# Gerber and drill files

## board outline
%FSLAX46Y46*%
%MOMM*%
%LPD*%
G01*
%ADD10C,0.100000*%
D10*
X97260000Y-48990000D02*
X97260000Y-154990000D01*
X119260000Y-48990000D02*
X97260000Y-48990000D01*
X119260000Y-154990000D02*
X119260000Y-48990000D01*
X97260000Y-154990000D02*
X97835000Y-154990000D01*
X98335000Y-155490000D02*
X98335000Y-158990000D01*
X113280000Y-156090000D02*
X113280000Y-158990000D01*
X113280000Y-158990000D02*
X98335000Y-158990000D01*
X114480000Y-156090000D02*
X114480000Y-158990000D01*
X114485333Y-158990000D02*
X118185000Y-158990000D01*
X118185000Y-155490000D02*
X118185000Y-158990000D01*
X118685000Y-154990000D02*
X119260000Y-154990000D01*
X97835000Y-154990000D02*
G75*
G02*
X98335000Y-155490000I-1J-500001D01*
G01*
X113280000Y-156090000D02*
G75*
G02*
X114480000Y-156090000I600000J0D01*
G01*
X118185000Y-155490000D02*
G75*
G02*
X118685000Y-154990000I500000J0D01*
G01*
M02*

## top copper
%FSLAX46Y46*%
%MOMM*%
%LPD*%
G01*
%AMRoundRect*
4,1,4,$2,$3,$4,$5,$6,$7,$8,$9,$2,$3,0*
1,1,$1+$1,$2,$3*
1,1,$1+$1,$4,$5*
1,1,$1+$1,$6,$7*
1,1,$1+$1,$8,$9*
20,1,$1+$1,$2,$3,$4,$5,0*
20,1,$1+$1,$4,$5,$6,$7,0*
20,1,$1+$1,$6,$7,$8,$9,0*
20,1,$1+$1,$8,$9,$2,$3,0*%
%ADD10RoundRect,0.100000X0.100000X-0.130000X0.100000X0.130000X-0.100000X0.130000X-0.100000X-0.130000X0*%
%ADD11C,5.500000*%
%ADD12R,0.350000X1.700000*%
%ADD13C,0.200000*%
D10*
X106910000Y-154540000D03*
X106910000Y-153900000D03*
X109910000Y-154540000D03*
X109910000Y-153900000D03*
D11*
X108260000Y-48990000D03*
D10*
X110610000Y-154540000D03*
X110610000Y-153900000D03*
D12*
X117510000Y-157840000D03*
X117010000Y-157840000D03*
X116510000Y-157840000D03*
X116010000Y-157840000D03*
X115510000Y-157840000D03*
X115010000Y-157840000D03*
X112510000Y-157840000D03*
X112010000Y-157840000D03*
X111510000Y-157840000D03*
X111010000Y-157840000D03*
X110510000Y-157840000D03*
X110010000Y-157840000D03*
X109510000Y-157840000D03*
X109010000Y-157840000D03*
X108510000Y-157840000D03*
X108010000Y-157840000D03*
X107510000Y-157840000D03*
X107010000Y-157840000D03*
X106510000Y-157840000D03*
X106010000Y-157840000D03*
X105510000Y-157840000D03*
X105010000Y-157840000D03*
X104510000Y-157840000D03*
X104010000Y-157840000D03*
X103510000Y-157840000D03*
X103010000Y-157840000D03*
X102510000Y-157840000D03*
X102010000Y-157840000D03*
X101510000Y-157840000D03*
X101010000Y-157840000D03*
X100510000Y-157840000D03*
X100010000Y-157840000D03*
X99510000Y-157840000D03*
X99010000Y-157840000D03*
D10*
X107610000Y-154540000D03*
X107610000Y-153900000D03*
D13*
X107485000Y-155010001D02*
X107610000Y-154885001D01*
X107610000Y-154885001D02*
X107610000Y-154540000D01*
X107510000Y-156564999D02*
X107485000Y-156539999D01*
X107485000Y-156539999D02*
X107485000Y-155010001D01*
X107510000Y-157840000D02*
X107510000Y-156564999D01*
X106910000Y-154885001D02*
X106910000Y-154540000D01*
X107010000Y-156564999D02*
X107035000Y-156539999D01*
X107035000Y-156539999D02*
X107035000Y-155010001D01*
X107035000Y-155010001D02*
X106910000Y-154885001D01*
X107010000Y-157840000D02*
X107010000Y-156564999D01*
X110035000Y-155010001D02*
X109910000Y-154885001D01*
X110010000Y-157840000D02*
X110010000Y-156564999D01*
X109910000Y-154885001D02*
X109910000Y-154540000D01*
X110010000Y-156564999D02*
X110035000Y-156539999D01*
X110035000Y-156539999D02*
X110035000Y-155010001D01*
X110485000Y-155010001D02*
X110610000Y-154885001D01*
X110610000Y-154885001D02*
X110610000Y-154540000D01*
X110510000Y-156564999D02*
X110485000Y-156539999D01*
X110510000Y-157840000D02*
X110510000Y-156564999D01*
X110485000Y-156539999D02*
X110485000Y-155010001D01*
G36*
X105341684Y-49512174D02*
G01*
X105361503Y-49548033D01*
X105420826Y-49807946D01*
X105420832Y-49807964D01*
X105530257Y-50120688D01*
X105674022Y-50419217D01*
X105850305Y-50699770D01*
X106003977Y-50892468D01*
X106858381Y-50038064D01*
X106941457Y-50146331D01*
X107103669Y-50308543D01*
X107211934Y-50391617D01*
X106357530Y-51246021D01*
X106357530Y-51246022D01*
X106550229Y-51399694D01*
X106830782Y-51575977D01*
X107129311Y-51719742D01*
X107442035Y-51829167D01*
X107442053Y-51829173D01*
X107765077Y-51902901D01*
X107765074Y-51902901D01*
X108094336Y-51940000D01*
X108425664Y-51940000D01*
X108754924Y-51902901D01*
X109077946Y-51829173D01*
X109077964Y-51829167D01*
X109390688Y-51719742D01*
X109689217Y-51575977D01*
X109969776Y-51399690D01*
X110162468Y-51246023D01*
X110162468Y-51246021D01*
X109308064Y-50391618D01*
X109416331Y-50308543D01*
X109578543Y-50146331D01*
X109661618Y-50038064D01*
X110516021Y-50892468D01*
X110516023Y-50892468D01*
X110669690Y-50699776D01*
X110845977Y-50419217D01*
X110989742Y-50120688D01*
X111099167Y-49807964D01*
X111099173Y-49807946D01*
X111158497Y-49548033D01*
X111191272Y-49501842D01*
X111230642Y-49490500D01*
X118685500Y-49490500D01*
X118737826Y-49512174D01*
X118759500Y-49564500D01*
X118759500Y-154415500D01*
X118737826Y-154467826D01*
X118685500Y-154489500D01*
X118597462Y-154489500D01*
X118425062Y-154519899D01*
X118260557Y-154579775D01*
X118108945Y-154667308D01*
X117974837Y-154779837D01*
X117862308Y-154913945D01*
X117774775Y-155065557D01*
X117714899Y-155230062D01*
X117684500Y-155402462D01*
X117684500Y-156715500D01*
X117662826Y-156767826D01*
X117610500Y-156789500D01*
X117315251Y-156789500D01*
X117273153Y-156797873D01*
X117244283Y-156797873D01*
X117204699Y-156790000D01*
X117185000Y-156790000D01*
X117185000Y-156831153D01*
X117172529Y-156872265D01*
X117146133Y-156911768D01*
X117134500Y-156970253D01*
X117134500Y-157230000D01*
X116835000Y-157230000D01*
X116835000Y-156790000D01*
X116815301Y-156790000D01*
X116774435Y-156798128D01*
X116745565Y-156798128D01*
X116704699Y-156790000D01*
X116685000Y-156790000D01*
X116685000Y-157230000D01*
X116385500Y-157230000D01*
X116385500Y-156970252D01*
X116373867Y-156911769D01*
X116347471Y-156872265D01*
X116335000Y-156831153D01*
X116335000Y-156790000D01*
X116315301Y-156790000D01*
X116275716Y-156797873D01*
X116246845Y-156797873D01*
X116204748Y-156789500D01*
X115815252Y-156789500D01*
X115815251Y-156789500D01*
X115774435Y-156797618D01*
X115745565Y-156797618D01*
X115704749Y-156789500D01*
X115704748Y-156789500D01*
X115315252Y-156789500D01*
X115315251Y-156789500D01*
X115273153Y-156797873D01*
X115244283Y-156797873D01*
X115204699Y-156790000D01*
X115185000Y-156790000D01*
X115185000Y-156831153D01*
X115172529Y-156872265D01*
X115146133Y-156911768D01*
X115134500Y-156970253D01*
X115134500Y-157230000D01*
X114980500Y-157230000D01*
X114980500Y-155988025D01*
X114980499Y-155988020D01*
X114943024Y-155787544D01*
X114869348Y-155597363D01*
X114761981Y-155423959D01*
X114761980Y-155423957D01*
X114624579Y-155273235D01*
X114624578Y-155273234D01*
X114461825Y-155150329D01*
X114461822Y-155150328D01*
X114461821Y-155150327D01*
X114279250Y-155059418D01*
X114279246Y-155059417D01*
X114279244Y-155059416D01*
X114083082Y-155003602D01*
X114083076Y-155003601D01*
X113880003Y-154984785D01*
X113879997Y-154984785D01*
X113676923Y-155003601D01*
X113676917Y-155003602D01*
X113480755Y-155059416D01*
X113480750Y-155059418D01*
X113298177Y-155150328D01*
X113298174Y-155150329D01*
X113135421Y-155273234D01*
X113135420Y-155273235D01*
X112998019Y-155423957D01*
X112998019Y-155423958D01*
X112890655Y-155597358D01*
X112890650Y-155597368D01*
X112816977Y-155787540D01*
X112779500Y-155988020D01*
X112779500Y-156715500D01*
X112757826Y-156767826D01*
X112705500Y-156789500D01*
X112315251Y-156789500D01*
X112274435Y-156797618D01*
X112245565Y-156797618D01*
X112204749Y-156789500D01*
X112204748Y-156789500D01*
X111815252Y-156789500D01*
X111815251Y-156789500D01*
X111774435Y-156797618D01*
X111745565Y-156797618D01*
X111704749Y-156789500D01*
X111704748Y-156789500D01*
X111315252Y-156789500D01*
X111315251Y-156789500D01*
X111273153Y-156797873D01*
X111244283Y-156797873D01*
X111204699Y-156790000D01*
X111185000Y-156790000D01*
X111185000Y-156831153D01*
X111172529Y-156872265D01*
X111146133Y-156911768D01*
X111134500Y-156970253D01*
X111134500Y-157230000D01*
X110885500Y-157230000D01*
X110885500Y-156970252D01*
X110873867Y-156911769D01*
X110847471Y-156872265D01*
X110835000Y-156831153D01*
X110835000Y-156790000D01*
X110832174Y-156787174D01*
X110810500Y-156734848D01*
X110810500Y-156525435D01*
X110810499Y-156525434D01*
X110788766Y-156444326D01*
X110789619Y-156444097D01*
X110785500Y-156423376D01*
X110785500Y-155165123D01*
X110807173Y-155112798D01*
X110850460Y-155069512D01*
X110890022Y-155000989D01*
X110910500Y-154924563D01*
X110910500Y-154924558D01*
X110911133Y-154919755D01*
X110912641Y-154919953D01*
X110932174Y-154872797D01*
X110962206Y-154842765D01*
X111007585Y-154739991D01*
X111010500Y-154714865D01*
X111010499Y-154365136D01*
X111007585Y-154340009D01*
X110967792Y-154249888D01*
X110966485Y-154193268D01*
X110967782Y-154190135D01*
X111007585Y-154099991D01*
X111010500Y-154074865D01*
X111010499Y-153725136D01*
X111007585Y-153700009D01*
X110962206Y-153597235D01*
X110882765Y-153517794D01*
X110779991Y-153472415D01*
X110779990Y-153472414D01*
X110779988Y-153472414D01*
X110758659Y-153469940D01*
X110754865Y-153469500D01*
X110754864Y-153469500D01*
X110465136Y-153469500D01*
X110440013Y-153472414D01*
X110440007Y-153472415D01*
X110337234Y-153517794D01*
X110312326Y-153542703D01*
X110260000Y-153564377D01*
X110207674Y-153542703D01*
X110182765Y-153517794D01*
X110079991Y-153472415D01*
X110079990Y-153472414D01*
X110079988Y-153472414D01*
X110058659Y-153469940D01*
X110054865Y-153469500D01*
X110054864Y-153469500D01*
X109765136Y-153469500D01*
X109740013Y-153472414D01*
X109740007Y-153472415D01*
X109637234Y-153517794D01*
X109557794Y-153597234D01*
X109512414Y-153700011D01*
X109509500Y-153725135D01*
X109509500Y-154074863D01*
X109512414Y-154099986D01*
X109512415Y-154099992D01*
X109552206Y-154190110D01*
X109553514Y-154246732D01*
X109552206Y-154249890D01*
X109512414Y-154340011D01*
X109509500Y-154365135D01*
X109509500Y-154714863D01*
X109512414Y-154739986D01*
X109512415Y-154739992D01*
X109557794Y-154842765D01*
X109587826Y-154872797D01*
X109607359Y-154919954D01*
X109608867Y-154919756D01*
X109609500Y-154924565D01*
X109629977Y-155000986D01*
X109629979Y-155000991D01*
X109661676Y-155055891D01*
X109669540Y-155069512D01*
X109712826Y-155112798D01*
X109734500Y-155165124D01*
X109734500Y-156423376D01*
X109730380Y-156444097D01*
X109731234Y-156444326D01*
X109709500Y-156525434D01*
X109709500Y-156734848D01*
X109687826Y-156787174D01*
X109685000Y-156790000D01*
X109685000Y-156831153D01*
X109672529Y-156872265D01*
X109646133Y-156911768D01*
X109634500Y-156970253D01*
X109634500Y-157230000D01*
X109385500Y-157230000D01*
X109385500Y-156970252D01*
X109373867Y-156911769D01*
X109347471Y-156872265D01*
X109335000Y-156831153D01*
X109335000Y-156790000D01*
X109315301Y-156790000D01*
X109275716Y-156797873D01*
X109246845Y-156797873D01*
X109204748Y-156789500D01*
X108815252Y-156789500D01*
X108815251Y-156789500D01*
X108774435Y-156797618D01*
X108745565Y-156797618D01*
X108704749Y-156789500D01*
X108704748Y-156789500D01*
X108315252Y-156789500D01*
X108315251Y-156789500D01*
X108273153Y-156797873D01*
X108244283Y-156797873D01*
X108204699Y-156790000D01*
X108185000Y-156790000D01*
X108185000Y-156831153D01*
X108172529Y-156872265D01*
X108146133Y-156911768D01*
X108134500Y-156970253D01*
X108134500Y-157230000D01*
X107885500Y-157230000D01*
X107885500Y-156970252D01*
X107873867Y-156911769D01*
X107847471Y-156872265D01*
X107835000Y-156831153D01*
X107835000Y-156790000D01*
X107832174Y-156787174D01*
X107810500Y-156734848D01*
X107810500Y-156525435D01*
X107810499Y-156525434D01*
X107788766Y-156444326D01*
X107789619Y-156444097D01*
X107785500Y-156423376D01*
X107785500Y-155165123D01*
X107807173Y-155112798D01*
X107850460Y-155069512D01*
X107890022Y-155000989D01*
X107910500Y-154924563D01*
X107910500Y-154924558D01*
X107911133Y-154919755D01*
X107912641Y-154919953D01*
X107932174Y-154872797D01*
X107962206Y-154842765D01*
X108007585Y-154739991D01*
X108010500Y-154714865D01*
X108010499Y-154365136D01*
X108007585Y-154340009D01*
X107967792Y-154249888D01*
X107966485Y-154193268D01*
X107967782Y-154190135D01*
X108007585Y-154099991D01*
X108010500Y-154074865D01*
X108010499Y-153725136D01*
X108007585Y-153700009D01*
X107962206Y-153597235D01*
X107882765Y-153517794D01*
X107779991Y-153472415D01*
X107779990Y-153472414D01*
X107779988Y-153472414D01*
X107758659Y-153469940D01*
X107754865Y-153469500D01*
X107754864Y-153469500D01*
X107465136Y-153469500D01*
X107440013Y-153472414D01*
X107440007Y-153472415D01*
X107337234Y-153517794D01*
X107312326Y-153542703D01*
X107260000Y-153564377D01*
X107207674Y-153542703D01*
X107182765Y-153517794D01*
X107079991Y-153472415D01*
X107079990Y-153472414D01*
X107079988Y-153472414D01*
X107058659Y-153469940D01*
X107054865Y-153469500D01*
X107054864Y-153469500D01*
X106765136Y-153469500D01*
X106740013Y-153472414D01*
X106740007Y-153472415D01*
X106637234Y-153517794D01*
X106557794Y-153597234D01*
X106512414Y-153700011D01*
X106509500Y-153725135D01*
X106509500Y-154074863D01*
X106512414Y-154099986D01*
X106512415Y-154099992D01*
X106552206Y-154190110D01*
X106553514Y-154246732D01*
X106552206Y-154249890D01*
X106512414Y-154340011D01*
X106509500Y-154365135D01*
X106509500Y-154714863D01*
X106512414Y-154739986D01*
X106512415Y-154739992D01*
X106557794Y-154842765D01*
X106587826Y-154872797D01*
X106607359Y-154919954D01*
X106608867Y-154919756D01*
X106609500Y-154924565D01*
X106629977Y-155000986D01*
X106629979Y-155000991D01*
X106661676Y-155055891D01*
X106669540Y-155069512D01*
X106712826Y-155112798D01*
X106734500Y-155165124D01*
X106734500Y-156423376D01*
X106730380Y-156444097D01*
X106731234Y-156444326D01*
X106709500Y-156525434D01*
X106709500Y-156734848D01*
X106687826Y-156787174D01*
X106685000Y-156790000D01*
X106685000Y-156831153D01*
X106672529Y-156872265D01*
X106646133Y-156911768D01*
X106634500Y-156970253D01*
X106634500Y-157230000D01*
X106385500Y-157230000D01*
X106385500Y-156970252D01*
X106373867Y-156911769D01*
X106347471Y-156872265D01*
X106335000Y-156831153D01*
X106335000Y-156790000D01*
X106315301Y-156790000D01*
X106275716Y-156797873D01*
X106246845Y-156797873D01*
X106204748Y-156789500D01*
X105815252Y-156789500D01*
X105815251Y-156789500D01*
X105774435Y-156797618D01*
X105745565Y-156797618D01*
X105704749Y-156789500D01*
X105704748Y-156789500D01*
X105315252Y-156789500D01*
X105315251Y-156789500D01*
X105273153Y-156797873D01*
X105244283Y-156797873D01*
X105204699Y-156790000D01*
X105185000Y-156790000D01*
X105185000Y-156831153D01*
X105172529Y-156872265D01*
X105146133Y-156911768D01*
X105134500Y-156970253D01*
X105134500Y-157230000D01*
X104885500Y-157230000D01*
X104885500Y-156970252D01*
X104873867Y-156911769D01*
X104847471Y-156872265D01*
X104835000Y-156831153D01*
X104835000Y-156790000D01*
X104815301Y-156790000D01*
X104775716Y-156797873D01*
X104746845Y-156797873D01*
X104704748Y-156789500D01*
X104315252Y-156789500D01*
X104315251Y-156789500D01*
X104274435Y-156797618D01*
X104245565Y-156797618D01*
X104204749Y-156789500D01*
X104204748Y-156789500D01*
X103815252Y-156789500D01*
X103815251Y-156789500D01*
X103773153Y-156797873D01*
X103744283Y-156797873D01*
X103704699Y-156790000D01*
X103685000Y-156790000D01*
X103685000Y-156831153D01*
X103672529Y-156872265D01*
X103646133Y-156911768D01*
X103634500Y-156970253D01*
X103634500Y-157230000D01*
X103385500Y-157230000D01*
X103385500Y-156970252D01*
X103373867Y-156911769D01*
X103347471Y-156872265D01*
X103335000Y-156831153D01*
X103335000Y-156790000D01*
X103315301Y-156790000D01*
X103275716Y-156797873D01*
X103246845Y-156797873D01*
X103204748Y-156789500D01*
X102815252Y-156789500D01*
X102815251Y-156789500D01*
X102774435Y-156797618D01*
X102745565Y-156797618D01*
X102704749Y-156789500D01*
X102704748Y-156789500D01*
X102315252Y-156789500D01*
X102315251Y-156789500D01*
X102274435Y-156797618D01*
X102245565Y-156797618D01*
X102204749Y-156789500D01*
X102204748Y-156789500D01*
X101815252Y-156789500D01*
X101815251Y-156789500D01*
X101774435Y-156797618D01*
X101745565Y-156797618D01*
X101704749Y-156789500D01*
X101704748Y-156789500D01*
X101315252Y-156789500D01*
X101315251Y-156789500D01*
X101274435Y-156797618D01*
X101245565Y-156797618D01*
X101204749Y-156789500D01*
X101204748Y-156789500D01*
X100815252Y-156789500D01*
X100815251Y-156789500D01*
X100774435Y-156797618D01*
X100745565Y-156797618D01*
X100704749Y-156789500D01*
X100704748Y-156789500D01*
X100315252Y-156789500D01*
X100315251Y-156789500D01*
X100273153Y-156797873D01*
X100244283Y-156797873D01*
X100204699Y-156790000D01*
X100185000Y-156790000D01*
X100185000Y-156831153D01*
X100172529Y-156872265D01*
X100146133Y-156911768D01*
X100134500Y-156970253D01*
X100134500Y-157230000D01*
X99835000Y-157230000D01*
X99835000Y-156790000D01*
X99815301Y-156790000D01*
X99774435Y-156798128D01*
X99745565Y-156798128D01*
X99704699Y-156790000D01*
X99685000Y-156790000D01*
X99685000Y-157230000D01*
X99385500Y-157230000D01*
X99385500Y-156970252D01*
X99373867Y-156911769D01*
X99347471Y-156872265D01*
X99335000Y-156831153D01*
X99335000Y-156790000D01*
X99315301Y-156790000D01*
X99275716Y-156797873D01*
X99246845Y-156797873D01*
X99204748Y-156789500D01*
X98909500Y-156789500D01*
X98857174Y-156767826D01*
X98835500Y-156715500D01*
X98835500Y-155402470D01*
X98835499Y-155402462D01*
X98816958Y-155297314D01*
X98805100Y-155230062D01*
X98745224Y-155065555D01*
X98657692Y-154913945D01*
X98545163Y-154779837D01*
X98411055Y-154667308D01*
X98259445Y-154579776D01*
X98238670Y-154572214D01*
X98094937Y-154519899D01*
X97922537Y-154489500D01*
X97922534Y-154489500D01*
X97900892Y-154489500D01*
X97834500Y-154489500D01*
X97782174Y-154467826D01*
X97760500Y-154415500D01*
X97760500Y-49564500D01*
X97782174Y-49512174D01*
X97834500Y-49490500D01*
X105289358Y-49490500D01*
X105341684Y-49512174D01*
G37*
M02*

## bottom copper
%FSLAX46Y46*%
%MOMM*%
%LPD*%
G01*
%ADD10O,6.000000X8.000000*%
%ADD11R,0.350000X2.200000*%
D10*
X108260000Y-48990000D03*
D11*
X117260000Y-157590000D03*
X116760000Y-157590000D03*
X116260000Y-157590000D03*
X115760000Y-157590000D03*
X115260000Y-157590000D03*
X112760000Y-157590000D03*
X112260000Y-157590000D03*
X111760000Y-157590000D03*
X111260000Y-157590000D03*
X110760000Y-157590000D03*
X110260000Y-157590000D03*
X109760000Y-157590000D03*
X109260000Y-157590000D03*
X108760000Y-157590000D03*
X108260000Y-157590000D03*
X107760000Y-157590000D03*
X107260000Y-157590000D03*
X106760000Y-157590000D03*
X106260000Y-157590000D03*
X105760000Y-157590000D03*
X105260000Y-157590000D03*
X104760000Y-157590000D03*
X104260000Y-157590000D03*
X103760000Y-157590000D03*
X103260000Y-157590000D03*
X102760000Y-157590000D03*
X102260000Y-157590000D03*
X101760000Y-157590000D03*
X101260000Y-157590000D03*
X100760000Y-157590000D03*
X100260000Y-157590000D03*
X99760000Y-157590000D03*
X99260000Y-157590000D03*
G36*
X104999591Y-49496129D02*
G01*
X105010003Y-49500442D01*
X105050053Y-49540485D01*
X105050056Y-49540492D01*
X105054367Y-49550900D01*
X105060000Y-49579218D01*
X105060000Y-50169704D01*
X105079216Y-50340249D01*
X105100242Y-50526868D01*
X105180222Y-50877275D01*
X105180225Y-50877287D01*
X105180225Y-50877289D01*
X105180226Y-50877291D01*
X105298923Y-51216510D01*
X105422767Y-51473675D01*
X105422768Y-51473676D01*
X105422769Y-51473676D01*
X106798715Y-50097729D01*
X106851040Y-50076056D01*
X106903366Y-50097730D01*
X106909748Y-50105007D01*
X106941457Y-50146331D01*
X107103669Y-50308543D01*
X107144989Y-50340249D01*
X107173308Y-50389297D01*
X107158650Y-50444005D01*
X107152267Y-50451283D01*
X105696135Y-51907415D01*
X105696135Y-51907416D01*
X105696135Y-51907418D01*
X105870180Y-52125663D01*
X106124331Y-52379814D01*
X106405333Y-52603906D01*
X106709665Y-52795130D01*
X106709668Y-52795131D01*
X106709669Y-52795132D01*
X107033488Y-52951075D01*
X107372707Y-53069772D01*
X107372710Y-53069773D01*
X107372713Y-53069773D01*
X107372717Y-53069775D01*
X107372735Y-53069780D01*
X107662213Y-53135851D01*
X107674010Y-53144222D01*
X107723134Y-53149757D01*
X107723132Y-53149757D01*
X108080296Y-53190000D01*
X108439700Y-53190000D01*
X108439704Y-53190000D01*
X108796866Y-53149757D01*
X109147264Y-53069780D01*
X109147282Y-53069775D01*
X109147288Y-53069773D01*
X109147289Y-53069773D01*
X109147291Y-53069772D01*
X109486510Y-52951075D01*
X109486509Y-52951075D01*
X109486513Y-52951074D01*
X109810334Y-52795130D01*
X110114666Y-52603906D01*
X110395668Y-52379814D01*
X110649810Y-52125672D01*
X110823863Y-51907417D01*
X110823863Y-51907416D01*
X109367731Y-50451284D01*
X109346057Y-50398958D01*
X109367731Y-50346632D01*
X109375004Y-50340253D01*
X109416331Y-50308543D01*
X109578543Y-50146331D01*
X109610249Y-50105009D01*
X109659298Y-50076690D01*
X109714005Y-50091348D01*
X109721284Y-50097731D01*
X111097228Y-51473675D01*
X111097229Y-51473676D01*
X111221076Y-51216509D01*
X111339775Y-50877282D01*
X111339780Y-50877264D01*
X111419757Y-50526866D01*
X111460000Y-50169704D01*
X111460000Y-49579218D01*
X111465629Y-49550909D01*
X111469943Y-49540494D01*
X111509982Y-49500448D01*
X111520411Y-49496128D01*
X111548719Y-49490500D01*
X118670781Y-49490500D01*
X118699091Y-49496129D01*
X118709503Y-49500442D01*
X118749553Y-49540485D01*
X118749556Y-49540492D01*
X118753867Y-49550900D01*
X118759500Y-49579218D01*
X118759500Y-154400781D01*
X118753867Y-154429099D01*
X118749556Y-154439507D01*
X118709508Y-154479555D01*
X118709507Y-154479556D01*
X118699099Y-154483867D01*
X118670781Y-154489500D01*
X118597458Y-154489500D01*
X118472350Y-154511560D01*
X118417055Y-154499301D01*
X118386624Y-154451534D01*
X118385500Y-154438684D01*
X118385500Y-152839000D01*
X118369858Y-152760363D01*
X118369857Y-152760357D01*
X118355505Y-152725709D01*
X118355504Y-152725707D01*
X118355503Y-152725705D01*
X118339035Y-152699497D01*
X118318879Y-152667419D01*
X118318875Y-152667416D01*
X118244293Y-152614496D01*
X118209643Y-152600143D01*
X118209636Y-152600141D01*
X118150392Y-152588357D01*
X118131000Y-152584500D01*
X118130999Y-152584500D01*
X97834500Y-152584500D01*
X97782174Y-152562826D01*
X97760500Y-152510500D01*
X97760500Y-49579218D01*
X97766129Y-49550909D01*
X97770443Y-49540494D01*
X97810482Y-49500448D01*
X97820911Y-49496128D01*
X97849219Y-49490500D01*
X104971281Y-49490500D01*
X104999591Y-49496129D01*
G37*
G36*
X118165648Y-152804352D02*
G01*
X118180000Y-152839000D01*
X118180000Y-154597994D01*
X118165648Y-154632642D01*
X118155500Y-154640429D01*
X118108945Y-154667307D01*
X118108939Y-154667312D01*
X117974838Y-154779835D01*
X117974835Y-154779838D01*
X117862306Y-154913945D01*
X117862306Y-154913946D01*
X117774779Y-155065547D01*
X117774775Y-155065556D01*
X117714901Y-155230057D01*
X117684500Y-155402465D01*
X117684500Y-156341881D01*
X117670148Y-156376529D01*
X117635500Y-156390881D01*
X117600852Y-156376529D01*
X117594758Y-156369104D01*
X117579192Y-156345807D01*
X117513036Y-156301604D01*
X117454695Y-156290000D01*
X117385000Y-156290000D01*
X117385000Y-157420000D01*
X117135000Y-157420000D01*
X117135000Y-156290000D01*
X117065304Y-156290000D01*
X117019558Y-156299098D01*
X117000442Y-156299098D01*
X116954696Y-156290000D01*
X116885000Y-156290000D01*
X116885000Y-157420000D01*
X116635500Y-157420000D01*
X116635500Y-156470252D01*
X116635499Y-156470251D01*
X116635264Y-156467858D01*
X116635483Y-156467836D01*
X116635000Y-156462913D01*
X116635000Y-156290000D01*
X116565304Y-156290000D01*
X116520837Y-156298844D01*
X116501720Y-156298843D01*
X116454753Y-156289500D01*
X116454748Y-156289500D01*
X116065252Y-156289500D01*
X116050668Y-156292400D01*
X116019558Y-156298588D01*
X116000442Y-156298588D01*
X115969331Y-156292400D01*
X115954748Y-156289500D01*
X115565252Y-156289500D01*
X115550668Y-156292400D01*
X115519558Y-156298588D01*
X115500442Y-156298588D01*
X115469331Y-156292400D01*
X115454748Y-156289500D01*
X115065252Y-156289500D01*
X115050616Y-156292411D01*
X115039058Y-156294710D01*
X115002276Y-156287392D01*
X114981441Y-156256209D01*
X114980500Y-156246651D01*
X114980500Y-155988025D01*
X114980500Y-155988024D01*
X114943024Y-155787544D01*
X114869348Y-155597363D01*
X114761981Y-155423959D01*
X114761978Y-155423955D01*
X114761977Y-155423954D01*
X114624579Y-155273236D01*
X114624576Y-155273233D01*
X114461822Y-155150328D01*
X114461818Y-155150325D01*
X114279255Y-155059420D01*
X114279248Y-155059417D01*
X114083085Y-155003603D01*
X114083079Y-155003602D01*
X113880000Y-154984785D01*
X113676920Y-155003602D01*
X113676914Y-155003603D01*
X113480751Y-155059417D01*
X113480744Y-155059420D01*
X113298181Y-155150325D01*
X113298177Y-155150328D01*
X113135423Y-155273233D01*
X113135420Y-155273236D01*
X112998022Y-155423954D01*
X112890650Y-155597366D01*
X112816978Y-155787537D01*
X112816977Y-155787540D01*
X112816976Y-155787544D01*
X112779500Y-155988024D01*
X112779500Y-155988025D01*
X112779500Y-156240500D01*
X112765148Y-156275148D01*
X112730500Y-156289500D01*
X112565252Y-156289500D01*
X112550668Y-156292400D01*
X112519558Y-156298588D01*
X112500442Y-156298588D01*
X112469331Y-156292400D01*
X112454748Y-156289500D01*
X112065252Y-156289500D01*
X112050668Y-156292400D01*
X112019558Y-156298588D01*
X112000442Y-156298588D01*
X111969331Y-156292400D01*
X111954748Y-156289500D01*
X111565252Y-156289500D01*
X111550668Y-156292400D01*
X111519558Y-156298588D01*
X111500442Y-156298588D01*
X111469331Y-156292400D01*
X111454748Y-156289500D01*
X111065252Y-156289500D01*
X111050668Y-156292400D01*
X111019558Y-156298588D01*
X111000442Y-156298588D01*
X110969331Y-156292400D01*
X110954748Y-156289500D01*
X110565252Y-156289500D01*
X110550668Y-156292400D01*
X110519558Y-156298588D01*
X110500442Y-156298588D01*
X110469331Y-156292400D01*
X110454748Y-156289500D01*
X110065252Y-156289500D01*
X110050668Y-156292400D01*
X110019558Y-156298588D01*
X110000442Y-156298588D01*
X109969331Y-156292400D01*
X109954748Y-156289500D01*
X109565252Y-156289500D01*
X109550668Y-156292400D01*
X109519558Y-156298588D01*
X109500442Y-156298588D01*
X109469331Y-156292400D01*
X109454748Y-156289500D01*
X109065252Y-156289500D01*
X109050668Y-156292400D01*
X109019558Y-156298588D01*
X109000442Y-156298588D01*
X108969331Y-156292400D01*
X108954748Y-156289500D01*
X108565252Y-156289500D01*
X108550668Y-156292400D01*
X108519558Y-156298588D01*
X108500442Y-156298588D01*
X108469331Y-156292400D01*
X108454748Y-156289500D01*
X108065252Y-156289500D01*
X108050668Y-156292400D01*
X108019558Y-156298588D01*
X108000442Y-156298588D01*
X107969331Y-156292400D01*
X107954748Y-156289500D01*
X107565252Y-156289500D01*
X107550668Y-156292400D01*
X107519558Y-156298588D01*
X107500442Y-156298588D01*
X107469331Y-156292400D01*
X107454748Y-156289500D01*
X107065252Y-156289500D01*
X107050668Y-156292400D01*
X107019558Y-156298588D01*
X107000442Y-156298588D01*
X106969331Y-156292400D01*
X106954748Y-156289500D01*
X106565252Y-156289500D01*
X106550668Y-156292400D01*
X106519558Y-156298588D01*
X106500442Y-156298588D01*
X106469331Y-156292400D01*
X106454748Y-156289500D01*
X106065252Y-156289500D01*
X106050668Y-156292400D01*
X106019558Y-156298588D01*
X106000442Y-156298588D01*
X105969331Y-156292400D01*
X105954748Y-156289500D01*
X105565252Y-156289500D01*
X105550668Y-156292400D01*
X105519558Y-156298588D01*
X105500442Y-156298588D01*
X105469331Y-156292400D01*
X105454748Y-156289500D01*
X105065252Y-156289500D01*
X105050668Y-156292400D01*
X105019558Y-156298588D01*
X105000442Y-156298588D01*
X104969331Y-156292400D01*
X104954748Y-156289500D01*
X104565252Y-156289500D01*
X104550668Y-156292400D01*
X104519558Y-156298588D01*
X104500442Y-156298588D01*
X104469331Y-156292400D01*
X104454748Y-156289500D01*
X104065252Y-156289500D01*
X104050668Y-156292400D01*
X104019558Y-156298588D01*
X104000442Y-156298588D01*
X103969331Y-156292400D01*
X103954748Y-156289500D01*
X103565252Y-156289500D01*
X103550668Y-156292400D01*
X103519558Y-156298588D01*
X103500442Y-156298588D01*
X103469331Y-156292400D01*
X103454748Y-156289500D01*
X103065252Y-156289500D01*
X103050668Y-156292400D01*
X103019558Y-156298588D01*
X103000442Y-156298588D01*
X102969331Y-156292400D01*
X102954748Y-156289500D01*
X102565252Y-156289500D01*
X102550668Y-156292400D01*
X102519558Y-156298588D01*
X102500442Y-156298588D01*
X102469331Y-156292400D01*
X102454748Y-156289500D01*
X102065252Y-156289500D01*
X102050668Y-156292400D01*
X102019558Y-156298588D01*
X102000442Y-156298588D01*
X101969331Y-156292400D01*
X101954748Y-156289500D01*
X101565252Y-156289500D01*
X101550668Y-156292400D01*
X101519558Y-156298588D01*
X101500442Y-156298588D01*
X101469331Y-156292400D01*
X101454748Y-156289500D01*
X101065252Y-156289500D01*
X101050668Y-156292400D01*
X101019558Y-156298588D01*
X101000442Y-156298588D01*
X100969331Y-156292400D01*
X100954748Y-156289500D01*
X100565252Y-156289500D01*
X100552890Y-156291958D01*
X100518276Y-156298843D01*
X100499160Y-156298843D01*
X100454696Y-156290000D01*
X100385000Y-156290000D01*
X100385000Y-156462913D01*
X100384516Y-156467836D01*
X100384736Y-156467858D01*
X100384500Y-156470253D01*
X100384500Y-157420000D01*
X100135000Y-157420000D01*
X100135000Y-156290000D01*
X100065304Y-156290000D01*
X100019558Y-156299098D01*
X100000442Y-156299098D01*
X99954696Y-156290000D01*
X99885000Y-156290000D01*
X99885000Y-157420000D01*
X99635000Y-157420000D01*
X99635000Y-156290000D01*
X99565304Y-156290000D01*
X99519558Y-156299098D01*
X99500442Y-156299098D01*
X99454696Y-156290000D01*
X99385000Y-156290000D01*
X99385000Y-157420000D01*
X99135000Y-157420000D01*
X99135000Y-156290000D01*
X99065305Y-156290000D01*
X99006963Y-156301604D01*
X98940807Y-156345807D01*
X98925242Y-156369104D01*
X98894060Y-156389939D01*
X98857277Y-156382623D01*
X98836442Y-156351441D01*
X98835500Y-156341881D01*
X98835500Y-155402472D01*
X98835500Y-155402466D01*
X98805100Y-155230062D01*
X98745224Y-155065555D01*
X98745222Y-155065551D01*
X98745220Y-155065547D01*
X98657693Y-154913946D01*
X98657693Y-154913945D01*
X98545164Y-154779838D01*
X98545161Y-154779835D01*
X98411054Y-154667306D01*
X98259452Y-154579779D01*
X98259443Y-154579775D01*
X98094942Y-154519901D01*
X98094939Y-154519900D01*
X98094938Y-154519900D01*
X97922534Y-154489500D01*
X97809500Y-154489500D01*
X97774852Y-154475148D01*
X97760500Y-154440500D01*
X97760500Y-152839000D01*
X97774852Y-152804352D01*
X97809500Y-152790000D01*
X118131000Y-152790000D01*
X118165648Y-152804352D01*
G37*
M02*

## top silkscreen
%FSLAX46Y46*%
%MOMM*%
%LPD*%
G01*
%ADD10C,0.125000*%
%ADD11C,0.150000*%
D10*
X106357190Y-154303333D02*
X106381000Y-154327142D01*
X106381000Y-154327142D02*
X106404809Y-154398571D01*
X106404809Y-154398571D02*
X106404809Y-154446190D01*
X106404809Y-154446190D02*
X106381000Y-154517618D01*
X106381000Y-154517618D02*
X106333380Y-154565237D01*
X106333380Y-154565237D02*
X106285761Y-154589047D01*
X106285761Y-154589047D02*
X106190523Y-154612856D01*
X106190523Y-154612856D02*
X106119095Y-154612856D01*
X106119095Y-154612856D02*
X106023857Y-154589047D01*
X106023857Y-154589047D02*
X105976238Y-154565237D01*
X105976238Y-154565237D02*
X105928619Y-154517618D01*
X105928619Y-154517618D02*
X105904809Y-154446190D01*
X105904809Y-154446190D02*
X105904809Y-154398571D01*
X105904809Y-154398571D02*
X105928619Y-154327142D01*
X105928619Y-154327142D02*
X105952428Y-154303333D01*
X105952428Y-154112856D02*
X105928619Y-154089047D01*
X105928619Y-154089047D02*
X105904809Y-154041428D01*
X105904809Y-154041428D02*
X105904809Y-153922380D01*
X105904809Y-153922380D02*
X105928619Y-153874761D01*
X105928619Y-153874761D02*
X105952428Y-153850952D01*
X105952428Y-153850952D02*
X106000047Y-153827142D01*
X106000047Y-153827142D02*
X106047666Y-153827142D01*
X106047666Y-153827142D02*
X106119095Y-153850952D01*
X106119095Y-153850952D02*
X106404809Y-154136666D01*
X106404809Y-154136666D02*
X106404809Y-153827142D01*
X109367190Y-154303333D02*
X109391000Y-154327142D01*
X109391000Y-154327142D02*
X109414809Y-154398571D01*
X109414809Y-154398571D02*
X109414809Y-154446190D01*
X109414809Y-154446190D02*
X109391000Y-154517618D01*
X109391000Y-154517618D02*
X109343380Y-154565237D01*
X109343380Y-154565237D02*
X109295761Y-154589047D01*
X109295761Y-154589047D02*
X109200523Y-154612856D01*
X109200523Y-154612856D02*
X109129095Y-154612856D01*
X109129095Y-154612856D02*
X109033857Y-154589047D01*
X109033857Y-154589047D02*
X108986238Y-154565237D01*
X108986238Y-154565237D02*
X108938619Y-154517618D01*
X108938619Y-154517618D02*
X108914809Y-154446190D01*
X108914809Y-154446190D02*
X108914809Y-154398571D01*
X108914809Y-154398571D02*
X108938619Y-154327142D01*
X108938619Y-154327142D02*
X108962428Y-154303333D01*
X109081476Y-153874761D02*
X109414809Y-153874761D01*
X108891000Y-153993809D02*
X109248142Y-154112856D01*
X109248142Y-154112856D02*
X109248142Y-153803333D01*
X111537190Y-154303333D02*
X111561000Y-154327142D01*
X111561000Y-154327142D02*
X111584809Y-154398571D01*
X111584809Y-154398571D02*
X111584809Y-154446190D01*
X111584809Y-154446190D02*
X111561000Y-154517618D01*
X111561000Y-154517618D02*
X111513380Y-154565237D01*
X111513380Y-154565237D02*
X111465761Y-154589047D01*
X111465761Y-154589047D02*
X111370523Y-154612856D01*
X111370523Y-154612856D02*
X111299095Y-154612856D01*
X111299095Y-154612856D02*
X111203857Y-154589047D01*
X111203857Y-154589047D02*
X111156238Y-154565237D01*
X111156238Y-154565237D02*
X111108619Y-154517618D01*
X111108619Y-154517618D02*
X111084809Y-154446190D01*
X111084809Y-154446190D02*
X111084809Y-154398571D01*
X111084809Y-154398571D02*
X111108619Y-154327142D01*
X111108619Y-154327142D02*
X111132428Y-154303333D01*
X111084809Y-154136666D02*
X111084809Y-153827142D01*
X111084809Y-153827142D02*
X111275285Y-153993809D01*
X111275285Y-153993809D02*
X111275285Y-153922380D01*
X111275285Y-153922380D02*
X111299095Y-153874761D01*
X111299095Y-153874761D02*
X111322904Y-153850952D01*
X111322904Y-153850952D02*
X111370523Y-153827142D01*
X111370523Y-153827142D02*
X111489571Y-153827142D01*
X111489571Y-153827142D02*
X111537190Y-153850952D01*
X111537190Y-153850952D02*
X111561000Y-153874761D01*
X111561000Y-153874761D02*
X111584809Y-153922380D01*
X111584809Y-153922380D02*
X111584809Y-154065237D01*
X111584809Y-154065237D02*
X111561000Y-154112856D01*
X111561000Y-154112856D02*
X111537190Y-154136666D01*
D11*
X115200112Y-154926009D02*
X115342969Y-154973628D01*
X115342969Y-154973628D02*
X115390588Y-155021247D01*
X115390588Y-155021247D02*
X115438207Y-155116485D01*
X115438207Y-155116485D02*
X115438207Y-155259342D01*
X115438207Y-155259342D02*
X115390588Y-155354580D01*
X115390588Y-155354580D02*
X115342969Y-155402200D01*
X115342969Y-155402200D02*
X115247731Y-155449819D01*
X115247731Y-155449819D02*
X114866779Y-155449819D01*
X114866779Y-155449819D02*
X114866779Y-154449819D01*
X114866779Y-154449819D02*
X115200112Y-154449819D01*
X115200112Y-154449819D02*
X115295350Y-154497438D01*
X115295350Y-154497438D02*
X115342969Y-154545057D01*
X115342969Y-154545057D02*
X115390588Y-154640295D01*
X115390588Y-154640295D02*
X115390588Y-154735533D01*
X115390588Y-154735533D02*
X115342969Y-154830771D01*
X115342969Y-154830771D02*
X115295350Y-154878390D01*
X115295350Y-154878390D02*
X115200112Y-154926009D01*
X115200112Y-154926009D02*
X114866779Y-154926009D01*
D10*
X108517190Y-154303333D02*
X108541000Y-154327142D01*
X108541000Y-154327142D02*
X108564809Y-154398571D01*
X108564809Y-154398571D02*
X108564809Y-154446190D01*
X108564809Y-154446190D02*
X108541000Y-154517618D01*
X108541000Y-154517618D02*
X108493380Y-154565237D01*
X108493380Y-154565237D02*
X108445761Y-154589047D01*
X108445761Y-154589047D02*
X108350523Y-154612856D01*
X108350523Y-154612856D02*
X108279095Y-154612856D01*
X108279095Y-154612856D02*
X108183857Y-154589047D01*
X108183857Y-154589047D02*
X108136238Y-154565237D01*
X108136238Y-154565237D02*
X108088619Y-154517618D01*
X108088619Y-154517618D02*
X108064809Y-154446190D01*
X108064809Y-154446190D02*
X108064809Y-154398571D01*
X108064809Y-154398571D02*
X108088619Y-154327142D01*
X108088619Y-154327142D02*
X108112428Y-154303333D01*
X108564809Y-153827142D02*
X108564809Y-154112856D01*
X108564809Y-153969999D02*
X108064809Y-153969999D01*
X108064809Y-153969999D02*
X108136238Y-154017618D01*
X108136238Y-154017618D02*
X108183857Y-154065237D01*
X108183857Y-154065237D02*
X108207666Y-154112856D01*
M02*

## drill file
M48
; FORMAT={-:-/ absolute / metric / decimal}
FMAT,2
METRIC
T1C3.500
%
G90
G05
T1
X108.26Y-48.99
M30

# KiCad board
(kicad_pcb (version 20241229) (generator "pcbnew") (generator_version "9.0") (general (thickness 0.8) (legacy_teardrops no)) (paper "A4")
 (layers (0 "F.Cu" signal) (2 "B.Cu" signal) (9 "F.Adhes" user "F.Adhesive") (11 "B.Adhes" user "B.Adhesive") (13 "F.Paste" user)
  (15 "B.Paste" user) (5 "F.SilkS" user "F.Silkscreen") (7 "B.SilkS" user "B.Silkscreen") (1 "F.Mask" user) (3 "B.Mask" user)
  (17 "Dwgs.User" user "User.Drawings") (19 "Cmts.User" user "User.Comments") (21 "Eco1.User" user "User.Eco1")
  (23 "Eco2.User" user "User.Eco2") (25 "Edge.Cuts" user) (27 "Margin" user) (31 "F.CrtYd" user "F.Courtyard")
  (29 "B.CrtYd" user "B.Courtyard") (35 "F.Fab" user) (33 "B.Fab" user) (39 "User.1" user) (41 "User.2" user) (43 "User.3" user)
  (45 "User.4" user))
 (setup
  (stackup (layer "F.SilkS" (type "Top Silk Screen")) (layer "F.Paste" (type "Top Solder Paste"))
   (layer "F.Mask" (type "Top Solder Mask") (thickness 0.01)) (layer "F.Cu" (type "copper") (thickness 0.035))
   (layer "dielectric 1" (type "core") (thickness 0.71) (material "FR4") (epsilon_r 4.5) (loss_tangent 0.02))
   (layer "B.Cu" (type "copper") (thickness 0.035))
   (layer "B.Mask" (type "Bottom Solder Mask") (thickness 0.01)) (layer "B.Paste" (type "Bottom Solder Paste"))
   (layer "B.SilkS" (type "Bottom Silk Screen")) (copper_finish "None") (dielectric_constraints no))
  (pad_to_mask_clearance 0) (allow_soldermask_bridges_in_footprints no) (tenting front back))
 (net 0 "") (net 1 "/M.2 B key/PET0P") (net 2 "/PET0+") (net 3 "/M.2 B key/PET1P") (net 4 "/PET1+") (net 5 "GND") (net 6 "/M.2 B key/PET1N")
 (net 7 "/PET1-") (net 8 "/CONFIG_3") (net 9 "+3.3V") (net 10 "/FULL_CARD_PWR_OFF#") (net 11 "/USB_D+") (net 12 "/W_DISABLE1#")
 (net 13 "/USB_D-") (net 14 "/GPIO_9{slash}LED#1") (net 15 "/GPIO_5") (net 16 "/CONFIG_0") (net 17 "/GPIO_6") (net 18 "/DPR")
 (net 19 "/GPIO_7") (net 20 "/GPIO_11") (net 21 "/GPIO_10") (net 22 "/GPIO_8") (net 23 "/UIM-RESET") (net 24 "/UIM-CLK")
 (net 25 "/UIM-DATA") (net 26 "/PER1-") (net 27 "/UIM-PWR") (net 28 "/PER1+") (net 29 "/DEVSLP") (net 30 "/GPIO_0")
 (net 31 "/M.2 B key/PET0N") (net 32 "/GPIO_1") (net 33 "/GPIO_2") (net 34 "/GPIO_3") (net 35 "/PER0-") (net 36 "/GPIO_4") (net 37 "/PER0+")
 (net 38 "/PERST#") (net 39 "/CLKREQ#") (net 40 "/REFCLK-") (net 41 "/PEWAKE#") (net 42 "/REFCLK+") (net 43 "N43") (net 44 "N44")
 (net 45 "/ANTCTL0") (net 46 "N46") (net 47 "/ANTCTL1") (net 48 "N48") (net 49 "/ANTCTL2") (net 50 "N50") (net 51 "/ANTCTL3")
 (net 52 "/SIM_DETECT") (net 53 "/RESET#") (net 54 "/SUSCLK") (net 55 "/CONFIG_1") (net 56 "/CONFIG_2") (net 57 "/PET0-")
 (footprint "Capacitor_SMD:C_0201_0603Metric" (layer "F.Cu") (at 106.91 154.22 90)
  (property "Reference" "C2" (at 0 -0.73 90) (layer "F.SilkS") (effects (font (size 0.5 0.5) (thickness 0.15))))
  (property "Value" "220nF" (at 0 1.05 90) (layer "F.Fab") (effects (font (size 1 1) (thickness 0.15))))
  (pad "" smd roundrect (at -0.345 0 90) (size 0.318 0.36) (layers "F.Paste") (roundrect_rratio 0.25))
  (pad "" smd roundrect (at 0.345 0 90) (size 0.318 0.36) (layers "F.Paste") (roundrect_rratio 0.25))
  (pad "1" smd roundrect (at -0.32 0 90) (size 0.46 0.4) (layers "F.Cu" "F.Mask") (roundrect_rratio 0.25) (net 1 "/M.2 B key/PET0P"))
  (pad "2" smd roundrect (at 0.32 0 90) (size 0.46 0.4) (layers "F.Cu" "F.Mask") (roundrect_rratio 0.25) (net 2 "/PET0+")))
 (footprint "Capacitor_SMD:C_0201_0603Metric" (layer "F.Cu") (at 109.91 154.22 90)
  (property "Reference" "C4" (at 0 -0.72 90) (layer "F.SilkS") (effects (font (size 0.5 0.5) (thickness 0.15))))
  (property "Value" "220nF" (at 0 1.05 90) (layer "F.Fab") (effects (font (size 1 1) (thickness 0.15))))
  (pad "" smd roundrect (at -0.345 0 90) (size 0.318 0.36) (layers "F.Paste") (roundrect_rratio 0.25))
  (pad "" smd roundrect (at 0.345 0 90) (size 0.318 0.36) (layers "F.Paste") (roundrect_rratio 0.25))
  (pad "1" smd roundrect (at -0.32 0 90) (size 0.46 0.4) (layers "F.Cu" "F.Mask") (roundrect_rratio 0.25) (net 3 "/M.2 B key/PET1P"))
  (pad "2" smd roundrect (at 0.32 0 90) (size 0.46 0.4) (layers "F.Cu" "F.Mask") (roundrect_rratio 0.25) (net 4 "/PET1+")))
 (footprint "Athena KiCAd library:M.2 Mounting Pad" (layer "F.Cu") (at 108.26 48.99)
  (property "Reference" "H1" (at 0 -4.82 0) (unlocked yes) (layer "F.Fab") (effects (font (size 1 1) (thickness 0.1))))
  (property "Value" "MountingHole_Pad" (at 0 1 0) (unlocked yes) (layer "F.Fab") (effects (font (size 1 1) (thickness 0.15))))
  (pad "1" thru_hole circle (at 0 0) (size 5.5 5.5) (drill 3.5) (layers "*.Cu" "*.Mask") (remove_unused_layers no) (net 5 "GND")
   (padstack (mode front_inner_back)
    (layer "Inner" (shape circle) (size 5.5 5.5) (zone_connect -1))
    (layer "B.Cu" (shape oval) (size 6 8) (thermal_bridge_angle 45) (zone_connect -1)))))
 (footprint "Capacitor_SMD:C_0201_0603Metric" (layer "F.Cu") (at 110.61 154.22 90)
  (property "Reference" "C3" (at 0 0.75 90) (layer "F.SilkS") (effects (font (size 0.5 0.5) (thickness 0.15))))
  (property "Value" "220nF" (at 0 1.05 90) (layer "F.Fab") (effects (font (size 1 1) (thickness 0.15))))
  (pad "" smd roundrect (at -0.345 0 90) (size 0.318 0.36) (layers "F.Paste") (roundrect_rratio 0.25))
  (pad "" smd roundrect (at 0.345 0 90) (size 0.318 0.36) (layers "F.Paste") (roundrect_rratio 0.25))
  (pad "1" smd roundrect (at -0.32 0 90) (size 0.46 0.4) (layers "F.Cu" "F.Mask") (roundrect_rratio 0.25) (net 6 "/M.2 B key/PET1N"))
  (pad "2" smd roundrect (at 0.32 0 90) (size 0.46 0.4) (layers "F.Cu" "F.Mask") (roundrect_rratio 0.25) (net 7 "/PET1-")))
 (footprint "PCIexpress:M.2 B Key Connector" (layer "F.Cu") (at 108.26 157.88)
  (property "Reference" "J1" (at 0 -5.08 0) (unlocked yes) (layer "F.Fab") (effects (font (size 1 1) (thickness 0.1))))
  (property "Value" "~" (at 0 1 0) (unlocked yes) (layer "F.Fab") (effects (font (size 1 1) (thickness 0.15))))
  (fp_line (start -11 -2.89) (end -10.425 -2.89) (stroke (width 0.1) (type default)) (layer "Edge.Cuts"))
  (fp_line (start -9.925 -2.39) (end -9.925 1.11) (stroke (width 0.1) (type default)) (layer "Edge.Cuts"))
  (fp_line (start 5.02 -1.79) (end 5.02 1.11) (stroke (width 0.1) (type default)) (layer "Edge.Cuts"))
  (fp_line (start 5.02 1.11) (end -9.925 1.11) (stroke (width 0.1) (type default)) (layer "Edge.Cuts"))
  (fp_line (start 6.22 -1.79) (end 6.22 1.11) (stroke (width 0.1) (type default)) (layer "Edge.Cuts"))
  (fp_line (start 6.225333 1.11) (end 9.925 1.11) (stroke (width 0.1) (type default)) (layer "Edge.Cuts"))
  (fp_line (start 9.925 -2.39) (end 9.925 1.11) (stroke (width 0.1) (type default)) (layer "Edge.Cuts"))
  (fp_line (start 10.425 -2.89) (end 11 -2.89) (stroke (width 0.1) (type default)) (layer "Edge.Cuts"))
  (fp_arc (start -10.425 -2.89) (mid -10.071447 -2.743553) (end -9.925 -2.39) (stroke (width 0.1) (type default)) (layer "Edge.Cuts"))
  (fp_arc (start 5.02 -1.79) (mid 5.62 -2.39) (end 6.22 -1.79) (stroke (width 0.1) (type default)) (layer "Edge.Cuts"))
  (fp_arc (start 9.925 -2.39) (mid 10.071447 -2.743553) (end 10.425 -2.89) (stroke (width 0.1) (type default)) (layer "Edge.Cuts"))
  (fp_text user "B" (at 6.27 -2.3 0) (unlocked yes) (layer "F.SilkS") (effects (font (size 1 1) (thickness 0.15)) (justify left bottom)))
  (pad "1" smd rect (at 9.25 -0.04 180) (size 0.35 1.7) (layers "F.Cu") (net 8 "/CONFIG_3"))
  (pad "2" smd rect (at 9 -0.29 180) (size 0.35 2.2) (layers "B.Cu") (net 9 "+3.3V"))
  (pad "3" smd rect (at 8.75 -0.04 180) (size 0.35 1.7) (layers "F.Cu") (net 5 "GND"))
  (pad "4" smd rect (at 8.5 -0.29 180) (size 0.35 2.2) (layers "B.Cu") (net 9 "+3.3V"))
  (pad "5" smd rect (at 8.25 -0.04 180) (size 0.35 1.7) (layers "F.Cu") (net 5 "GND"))
  (pad "6" smd rect (at 8 -0.29 180) (size 0.35 2.2) (layers "B.Cu") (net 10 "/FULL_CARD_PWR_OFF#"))
  (pad "7" smd rect (at 7.75 -0.04 180) (size 0.35 1.7) (layers "F.Cu") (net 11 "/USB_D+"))
  (pad "8" smd rect (at 7.5 -0.29 180) (size 0.35 2.2) (layers "B.Cu") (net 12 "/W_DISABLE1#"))
  (pad "9" smd rect (at 7.25 -0.04 180) (size 0.35 1.7) (layers "F.Cu") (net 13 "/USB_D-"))
  (pad "10" smd rect (at 7 -0.29 180) (size 0.35 2.2) (layers "B.Cu") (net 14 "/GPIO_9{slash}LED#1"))
  (pad "11" smd rect (at 6.75 -0.04 180) (size 0.35 1.7) (layers "F.Cu") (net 5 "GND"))
  (pad "20" smd rect (at 4.5 -0.29 180) (size 0.35 2.2) (layers "B.Cu") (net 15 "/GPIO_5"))
  (pad "21" smd rect (at 4.25 -0.04 180) (size 0.35 1.7) (layers "F.Cu") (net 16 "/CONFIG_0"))
  (pad "22" smd rect (at 4 -0.29 180) (size 0.35 2.2) (layers "B.Cu") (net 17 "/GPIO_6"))
  (pad "23" smd rect (at 3.75 -0.04 180) (size 0.35 1.7) (layers "F.Cu") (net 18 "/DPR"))
  (pad "24" smd rect (at 3.5 -0.29 180) (size 0.35 2.2) (layers "B.Cu") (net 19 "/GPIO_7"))
  (pad "25" smd rect (at 3.25 -0.04 180) (size 0.35 1.7) (layers "F.Cu") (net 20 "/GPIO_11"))
  (pad "26" smd rect (at 3 -0.29 180) (size 0.35 2.2) (layers "B.Cu") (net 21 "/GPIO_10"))
  (pad "27" smd rect (at 2.75 -0.04 180) (size 0.35 1.7) (layers "F.Cu") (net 5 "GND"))
  (pad "28" smd rect (at 2.5 -0.29 180) (size 0.35 2.2) (layers "B.Cu") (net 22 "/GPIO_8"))
  (pad "29" smd rect (at 2.25 -0.04 180) (size 0.35 1.7) (layers "F.Cu") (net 6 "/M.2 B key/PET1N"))
  (pad "30" smd rect (at 2 -0.29 180) (size 0.35 2.2) (layers "B.Cu") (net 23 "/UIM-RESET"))
  (pad "31" smd rect (at 1.75 -0.04 180) (size 0.35 1.7) (layers "F.Cu") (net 3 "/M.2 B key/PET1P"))
  (pad "32" smd rect (at 1.5 -0.29 180) (size 0.35 2.2) (layers "B.Cu") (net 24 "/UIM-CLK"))
  (pad "33" smd rect (at 1.25 -0.04 180) (size 0.35 1.7) (layers "F.Cu") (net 5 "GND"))
  (pad "34" smd rect (at 1 -0.29 180) (size 0.35 2.2) (layers "B.Cu") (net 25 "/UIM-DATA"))
  (pad "35" smd rect (at 0.75 -0.04 180) (size 0.35 1.7) (layers "F.Cu") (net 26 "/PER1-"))
  (pad "36" smd rect (at 0.5 -0.29 180) (size 0.35 2.2) (layers "B.Cu") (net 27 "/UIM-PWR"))
  (pad "37" smd rect (at 0.25 -0.04 180) (size 0.35 1.7) (layers "F.Cu") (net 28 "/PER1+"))
  (pad "38" smd rect (at 0 -0.29 180) (size 0.35 2.2) (layers "B.Cu") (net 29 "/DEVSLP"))
  (pad "39" smd rect (at -0.25 -0.04 180) (size 0.35 1.7) (layers "F.Cu") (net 5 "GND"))
  (pad "40" smd rect (at -0.5 -0.29 180) (size 0.35 2.2) (layers "B.Cu") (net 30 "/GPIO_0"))
  (pad "41" smd rect (at -0.75 -0.04 180) (size 0.35 1.7) (layers "F.Cu") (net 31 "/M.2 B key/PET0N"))
  (pad "42" smd rect (at -1 -0.29 180) (size 0.35 2.2) (layers "B.Cu") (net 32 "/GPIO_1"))
  (pad "43" smd rect (at -1.25 -0.04 180) (size 0.35 1.7) (layers "F.Cu") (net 1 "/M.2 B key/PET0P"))
  (pad "44" smd rect (at -1.5 -0.29 180) (size 0.35 2.2) (layers "B.Cu") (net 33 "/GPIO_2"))
  (pad "45" smd rect (at -1.75 -0.04 180) (size 0.35 1.7) (layers "F.Cu") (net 5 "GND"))
  (pad "46" smd rect (at -2 -0.29 180) (size 0.35 2.2) (layers "B.Cu") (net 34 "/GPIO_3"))
  (pad "47" smd rect (at -2.25 -0.04 180) (size 0.35 1.7) (layers "F.Cu") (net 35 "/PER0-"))
  (pad "48" smd rect (at -2.5 -0.29 180) (size 0.35 2.2) (layers "B.Cu") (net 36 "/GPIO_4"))
  (pad "49" smd rect (at -2.75 -0.04 180) (size 0.35 1.7) (layers "F.Cu") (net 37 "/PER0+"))
  (pad "50" smd rect (at -3 -0.29 180) (size 0.35 2.2) (layers "B.Cu") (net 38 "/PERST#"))
  (pad "51" smd rect (at -3.25 -0.04 180) (size 0.35 1.7) (layers "F.Cu") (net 5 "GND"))
  (pad "52" smd rect (at -3.5 -0.29 180) (size 0.35 2.2) (layers "B.Cu") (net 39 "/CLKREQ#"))
  (pad "53" smd rect (at -3.75 -0.04 180) (size 0.35 1.7) (layers "F.Cu") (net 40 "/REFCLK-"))
  (pad "54" smd rect (at -4 -0.29 180) (size 0.35 2.2) (layers "B.Cu") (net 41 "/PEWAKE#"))
  (pad "55" smd rect (at -4.25 -0.04 180) (size 0.35 1.7) (layers "F.Cu") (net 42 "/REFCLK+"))
  (pad "56" smd rect (at -4.5 -0.29 180) (size 0.35 2.2) (layers "B.Cu") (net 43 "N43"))
  (pad "57" smd rect (at -4.75 -0.04 180) (size 0.35 1.7) (layers "F.Cu") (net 5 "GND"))
  (pad "58" smd rect (at -5 -0.29 180) (size 0.35 2.2) (layers "B.Cu") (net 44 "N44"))
  (pad "59" smd rect (at -5.25 -0.04 180) (size 0.35 1.7) (layers "F.Cu") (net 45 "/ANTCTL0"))
  (pad "60" smd rect (at -5.5 -0.29 180) (size 0.35 2.2) (layers "B.Cu") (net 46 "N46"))
  (pad "61" smd rect (at -5.75 -0.04 180) (size 0.35 1.7) (layers "F.Cu") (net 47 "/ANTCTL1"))
  (pad "62" smd rect (at -6 -0.29 180) (size 0.35 2.2) (layers "B.Cu") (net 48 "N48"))
  (pad "63" smd rect (at -6.25 -0.04 180) (size 0.35 1.7) (layers "F.Cu") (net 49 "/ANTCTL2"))
  (pad "64" smd rect (at -6.5 -0.29 180) (size 0.35 2.2) (layers "B.Cu") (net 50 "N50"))
  (pad "65" smd rect (at -6.75 -0.04 180) (size 0.35 1.7) (layers "F.Cu") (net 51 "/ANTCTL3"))
  (pad "66" smd rect (at -7 -0.29 180) (size 0.35 2.2) (layers "B.Cu") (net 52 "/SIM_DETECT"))
  (pad "67" smd rect (at -7.25 -0.04 180) (size 0.35 1.7) (layers "F.Cu") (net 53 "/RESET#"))
  (pad "68" smd rect (at -7.5 -0.29 180) (size 0.35 2.2) (layers "B.Cu") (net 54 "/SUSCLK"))
  (pad "69" smd rect (at -7.75 -0.04 180) (size 0.35 1.7) (layers "F.Cu") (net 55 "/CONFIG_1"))
  (pad "70" smd rect (at -8 -0.29 180) (size 0.35 2.2) (layers "B.Cu") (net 9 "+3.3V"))
  (pad "71" smd rect (at -8.25 -0.04 180) (size 0.35 1.7) (layers "F.Cu") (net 5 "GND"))
  (pad "72" smd rect (at -8.5 -0.29 180) (size 0.35 2.2) (layers "B.Cu") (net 9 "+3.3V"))
  (pad "73" smd rect (at -8.75 -0.04 180) (size 0.35 1.7) (layers "F.Cu") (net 5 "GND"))
  (pad "74" smd rect (at -9 -0.29 180) (size 0.35 2.2) (layers "B.Cu") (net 9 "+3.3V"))
  (pad "75" smd rect (at -9.25 -0.04 180) (size 0.35 1.7) (layers "F.Cu") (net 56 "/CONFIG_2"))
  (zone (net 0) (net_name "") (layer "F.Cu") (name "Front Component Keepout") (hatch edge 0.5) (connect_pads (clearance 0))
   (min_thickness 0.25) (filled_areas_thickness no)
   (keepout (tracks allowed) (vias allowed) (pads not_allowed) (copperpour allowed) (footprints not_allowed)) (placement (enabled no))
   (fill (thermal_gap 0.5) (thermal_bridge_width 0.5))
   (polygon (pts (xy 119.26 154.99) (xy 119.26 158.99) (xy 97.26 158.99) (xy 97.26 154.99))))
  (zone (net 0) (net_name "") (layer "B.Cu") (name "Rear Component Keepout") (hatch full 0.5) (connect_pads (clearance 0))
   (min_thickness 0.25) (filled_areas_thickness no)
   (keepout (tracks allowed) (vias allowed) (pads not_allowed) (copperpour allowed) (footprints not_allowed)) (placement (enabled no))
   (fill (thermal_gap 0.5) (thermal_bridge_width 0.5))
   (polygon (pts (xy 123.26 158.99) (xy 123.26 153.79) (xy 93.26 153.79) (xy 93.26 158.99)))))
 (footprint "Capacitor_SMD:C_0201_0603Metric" (layer "F.Cu") (at 107.61 154.22 90)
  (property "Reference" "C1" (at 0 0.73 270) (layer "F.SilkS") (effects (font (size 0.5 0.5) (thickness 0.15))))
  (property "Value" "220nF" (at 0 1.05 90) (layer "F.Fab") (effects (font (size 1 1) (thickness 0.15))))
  (pad "" smd roundrect (at -0.345 0 90) (size 0.318 0.36) (layers "F.Paste") (roundrect_rratio 0.25))
  (pad "" smd roundrect (at 0.345 0 90) (size 0.318 0.36) (layers "F.Paste") (roundrect_rratio 0.25))
  (pad "1" smd roundrect (at -0.32 0 90) (size 0.46 0.4) (layers "F.Cu" "F.Mask") (roundrect_rratio 0.25) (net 31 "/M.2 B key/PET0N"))
  (pad "2" smd roundrect (at 0.32 0 90) (size 0.46 0.4) (layers "F.Cu" "F.Mask") (roundrect_rratio 0.25) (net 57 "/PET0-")))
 (gr_line (start 97.26 48.99) (end 97.26 154.99) (stroke (width 0.1) (type default)) (layer "Edge.Cuts"))
 (gr_line (start 119.26 48.99) (end 97.26 48.99) (stroke (width 0.1) (type default)) (layer "Edge.Cuts"))
 (gr_line (start 119.26 154.99) (end 119.26 48.99) (stroke (width 0.1) (type default)) (layer "Edge.Cuts"))
 (segment (start 107.485 155.010001) (end 107.61 154.885001) (width 0.2) (layer "F.Cu") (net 31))
 (segment (start 107.61 154.885001) (end 107.61 154.54) (width 0.2) (layer "F.Cu") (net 31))
 (segment (start 107.51 156.564999) (end 107.485 156.539999) (width 0.2) (layer "F.Cu") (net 31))
 (segment (start 107.485 156.539999) (end 107.485 155.010001) (width 0.2) (layer "F.Cu") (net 31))
 (segment (start 107.51 157.84) (end 107.51 156.564999) (width 0.2) (layer "F.Cu") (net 31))
 (segment (start 106.91 154.885001) (end 106.91 154.54) (width 0.2) (layer "F.Cu") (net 1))
 (segment (start 107.01 156.564999) (end 107.035 156.539999) (width 0.2) (layer "F.Cu") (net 1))
 (segment (start 107.035 156.539999) (end 107.035 155.010001) (width 0.2) (layer "F.Cu") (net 1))
 (segment (start 107.035 155.010001) (end 106.91 154.885001) (width 0.2) (layer "F.Cu") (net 1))
 (segment (start 107.01 157.84) (end 107.01 156.564999) (width 0.2) (layer "F.Cu") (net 1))
 (segment (start 110.035 155.010001) (end 109.91 154.885001) (width 0.2) (layer "F.Cu") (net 3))
 (segment (start 110.01 157.84) (end 110.01 156.564999) (width 0.2) (layer "F.Cu") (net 3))
 (segment (start 109.91 154.885001) (end 109.91 154.54) (width 0.2) (layer "F.Cu") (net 3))
 (segment (start 110.01 156.564999) (end 110.035 156.539999) (width 0.2) (layer "F.Cu") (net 3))
 (segment (start 110.035 156.539999) (end 110.035 155.010001) (width 0.2) (layer "F.Cu") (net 3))
 (segment (start 110.485 155.010001) (end 110.61 154.885001) (width 0.2) (layer "F.Cu") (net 6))
 (segment (start 110.61 154.885001) (end 110.61 154.54) (width 0.2) (layer "F.Cu") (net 6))
 (segment (start 110.51 156.564999) (end 110.485 156.539999) (width 0.2) (layer "F.Cu") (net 6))
 (segment (start 110.51 157.84) (end 110.51 156.564999) (width 0.2) (layer "F.Cu") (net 6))
 (segment (start 110.485 156.539999) (end 110.485 155.010001) (width 0.2) (layer "F.Cu") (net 6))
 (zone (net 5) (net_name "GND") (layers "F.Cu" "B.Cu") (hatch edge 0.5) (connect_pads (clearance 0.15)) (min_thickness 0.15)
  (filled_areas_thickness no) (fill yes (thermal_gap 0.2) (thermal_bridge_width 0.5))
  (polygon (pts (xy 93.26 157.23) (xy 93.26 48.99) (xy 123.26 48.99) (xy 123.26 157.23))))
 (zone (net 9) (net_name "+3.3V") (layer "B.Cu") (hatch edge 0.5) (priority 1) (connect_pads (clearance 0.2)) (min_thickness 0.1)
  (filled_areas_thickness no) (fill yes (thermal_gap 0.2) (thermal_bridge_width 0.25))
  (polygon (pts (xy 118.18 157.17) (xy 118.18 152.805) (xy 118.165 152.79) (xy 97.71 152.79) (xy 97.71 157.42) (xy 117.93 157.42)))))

